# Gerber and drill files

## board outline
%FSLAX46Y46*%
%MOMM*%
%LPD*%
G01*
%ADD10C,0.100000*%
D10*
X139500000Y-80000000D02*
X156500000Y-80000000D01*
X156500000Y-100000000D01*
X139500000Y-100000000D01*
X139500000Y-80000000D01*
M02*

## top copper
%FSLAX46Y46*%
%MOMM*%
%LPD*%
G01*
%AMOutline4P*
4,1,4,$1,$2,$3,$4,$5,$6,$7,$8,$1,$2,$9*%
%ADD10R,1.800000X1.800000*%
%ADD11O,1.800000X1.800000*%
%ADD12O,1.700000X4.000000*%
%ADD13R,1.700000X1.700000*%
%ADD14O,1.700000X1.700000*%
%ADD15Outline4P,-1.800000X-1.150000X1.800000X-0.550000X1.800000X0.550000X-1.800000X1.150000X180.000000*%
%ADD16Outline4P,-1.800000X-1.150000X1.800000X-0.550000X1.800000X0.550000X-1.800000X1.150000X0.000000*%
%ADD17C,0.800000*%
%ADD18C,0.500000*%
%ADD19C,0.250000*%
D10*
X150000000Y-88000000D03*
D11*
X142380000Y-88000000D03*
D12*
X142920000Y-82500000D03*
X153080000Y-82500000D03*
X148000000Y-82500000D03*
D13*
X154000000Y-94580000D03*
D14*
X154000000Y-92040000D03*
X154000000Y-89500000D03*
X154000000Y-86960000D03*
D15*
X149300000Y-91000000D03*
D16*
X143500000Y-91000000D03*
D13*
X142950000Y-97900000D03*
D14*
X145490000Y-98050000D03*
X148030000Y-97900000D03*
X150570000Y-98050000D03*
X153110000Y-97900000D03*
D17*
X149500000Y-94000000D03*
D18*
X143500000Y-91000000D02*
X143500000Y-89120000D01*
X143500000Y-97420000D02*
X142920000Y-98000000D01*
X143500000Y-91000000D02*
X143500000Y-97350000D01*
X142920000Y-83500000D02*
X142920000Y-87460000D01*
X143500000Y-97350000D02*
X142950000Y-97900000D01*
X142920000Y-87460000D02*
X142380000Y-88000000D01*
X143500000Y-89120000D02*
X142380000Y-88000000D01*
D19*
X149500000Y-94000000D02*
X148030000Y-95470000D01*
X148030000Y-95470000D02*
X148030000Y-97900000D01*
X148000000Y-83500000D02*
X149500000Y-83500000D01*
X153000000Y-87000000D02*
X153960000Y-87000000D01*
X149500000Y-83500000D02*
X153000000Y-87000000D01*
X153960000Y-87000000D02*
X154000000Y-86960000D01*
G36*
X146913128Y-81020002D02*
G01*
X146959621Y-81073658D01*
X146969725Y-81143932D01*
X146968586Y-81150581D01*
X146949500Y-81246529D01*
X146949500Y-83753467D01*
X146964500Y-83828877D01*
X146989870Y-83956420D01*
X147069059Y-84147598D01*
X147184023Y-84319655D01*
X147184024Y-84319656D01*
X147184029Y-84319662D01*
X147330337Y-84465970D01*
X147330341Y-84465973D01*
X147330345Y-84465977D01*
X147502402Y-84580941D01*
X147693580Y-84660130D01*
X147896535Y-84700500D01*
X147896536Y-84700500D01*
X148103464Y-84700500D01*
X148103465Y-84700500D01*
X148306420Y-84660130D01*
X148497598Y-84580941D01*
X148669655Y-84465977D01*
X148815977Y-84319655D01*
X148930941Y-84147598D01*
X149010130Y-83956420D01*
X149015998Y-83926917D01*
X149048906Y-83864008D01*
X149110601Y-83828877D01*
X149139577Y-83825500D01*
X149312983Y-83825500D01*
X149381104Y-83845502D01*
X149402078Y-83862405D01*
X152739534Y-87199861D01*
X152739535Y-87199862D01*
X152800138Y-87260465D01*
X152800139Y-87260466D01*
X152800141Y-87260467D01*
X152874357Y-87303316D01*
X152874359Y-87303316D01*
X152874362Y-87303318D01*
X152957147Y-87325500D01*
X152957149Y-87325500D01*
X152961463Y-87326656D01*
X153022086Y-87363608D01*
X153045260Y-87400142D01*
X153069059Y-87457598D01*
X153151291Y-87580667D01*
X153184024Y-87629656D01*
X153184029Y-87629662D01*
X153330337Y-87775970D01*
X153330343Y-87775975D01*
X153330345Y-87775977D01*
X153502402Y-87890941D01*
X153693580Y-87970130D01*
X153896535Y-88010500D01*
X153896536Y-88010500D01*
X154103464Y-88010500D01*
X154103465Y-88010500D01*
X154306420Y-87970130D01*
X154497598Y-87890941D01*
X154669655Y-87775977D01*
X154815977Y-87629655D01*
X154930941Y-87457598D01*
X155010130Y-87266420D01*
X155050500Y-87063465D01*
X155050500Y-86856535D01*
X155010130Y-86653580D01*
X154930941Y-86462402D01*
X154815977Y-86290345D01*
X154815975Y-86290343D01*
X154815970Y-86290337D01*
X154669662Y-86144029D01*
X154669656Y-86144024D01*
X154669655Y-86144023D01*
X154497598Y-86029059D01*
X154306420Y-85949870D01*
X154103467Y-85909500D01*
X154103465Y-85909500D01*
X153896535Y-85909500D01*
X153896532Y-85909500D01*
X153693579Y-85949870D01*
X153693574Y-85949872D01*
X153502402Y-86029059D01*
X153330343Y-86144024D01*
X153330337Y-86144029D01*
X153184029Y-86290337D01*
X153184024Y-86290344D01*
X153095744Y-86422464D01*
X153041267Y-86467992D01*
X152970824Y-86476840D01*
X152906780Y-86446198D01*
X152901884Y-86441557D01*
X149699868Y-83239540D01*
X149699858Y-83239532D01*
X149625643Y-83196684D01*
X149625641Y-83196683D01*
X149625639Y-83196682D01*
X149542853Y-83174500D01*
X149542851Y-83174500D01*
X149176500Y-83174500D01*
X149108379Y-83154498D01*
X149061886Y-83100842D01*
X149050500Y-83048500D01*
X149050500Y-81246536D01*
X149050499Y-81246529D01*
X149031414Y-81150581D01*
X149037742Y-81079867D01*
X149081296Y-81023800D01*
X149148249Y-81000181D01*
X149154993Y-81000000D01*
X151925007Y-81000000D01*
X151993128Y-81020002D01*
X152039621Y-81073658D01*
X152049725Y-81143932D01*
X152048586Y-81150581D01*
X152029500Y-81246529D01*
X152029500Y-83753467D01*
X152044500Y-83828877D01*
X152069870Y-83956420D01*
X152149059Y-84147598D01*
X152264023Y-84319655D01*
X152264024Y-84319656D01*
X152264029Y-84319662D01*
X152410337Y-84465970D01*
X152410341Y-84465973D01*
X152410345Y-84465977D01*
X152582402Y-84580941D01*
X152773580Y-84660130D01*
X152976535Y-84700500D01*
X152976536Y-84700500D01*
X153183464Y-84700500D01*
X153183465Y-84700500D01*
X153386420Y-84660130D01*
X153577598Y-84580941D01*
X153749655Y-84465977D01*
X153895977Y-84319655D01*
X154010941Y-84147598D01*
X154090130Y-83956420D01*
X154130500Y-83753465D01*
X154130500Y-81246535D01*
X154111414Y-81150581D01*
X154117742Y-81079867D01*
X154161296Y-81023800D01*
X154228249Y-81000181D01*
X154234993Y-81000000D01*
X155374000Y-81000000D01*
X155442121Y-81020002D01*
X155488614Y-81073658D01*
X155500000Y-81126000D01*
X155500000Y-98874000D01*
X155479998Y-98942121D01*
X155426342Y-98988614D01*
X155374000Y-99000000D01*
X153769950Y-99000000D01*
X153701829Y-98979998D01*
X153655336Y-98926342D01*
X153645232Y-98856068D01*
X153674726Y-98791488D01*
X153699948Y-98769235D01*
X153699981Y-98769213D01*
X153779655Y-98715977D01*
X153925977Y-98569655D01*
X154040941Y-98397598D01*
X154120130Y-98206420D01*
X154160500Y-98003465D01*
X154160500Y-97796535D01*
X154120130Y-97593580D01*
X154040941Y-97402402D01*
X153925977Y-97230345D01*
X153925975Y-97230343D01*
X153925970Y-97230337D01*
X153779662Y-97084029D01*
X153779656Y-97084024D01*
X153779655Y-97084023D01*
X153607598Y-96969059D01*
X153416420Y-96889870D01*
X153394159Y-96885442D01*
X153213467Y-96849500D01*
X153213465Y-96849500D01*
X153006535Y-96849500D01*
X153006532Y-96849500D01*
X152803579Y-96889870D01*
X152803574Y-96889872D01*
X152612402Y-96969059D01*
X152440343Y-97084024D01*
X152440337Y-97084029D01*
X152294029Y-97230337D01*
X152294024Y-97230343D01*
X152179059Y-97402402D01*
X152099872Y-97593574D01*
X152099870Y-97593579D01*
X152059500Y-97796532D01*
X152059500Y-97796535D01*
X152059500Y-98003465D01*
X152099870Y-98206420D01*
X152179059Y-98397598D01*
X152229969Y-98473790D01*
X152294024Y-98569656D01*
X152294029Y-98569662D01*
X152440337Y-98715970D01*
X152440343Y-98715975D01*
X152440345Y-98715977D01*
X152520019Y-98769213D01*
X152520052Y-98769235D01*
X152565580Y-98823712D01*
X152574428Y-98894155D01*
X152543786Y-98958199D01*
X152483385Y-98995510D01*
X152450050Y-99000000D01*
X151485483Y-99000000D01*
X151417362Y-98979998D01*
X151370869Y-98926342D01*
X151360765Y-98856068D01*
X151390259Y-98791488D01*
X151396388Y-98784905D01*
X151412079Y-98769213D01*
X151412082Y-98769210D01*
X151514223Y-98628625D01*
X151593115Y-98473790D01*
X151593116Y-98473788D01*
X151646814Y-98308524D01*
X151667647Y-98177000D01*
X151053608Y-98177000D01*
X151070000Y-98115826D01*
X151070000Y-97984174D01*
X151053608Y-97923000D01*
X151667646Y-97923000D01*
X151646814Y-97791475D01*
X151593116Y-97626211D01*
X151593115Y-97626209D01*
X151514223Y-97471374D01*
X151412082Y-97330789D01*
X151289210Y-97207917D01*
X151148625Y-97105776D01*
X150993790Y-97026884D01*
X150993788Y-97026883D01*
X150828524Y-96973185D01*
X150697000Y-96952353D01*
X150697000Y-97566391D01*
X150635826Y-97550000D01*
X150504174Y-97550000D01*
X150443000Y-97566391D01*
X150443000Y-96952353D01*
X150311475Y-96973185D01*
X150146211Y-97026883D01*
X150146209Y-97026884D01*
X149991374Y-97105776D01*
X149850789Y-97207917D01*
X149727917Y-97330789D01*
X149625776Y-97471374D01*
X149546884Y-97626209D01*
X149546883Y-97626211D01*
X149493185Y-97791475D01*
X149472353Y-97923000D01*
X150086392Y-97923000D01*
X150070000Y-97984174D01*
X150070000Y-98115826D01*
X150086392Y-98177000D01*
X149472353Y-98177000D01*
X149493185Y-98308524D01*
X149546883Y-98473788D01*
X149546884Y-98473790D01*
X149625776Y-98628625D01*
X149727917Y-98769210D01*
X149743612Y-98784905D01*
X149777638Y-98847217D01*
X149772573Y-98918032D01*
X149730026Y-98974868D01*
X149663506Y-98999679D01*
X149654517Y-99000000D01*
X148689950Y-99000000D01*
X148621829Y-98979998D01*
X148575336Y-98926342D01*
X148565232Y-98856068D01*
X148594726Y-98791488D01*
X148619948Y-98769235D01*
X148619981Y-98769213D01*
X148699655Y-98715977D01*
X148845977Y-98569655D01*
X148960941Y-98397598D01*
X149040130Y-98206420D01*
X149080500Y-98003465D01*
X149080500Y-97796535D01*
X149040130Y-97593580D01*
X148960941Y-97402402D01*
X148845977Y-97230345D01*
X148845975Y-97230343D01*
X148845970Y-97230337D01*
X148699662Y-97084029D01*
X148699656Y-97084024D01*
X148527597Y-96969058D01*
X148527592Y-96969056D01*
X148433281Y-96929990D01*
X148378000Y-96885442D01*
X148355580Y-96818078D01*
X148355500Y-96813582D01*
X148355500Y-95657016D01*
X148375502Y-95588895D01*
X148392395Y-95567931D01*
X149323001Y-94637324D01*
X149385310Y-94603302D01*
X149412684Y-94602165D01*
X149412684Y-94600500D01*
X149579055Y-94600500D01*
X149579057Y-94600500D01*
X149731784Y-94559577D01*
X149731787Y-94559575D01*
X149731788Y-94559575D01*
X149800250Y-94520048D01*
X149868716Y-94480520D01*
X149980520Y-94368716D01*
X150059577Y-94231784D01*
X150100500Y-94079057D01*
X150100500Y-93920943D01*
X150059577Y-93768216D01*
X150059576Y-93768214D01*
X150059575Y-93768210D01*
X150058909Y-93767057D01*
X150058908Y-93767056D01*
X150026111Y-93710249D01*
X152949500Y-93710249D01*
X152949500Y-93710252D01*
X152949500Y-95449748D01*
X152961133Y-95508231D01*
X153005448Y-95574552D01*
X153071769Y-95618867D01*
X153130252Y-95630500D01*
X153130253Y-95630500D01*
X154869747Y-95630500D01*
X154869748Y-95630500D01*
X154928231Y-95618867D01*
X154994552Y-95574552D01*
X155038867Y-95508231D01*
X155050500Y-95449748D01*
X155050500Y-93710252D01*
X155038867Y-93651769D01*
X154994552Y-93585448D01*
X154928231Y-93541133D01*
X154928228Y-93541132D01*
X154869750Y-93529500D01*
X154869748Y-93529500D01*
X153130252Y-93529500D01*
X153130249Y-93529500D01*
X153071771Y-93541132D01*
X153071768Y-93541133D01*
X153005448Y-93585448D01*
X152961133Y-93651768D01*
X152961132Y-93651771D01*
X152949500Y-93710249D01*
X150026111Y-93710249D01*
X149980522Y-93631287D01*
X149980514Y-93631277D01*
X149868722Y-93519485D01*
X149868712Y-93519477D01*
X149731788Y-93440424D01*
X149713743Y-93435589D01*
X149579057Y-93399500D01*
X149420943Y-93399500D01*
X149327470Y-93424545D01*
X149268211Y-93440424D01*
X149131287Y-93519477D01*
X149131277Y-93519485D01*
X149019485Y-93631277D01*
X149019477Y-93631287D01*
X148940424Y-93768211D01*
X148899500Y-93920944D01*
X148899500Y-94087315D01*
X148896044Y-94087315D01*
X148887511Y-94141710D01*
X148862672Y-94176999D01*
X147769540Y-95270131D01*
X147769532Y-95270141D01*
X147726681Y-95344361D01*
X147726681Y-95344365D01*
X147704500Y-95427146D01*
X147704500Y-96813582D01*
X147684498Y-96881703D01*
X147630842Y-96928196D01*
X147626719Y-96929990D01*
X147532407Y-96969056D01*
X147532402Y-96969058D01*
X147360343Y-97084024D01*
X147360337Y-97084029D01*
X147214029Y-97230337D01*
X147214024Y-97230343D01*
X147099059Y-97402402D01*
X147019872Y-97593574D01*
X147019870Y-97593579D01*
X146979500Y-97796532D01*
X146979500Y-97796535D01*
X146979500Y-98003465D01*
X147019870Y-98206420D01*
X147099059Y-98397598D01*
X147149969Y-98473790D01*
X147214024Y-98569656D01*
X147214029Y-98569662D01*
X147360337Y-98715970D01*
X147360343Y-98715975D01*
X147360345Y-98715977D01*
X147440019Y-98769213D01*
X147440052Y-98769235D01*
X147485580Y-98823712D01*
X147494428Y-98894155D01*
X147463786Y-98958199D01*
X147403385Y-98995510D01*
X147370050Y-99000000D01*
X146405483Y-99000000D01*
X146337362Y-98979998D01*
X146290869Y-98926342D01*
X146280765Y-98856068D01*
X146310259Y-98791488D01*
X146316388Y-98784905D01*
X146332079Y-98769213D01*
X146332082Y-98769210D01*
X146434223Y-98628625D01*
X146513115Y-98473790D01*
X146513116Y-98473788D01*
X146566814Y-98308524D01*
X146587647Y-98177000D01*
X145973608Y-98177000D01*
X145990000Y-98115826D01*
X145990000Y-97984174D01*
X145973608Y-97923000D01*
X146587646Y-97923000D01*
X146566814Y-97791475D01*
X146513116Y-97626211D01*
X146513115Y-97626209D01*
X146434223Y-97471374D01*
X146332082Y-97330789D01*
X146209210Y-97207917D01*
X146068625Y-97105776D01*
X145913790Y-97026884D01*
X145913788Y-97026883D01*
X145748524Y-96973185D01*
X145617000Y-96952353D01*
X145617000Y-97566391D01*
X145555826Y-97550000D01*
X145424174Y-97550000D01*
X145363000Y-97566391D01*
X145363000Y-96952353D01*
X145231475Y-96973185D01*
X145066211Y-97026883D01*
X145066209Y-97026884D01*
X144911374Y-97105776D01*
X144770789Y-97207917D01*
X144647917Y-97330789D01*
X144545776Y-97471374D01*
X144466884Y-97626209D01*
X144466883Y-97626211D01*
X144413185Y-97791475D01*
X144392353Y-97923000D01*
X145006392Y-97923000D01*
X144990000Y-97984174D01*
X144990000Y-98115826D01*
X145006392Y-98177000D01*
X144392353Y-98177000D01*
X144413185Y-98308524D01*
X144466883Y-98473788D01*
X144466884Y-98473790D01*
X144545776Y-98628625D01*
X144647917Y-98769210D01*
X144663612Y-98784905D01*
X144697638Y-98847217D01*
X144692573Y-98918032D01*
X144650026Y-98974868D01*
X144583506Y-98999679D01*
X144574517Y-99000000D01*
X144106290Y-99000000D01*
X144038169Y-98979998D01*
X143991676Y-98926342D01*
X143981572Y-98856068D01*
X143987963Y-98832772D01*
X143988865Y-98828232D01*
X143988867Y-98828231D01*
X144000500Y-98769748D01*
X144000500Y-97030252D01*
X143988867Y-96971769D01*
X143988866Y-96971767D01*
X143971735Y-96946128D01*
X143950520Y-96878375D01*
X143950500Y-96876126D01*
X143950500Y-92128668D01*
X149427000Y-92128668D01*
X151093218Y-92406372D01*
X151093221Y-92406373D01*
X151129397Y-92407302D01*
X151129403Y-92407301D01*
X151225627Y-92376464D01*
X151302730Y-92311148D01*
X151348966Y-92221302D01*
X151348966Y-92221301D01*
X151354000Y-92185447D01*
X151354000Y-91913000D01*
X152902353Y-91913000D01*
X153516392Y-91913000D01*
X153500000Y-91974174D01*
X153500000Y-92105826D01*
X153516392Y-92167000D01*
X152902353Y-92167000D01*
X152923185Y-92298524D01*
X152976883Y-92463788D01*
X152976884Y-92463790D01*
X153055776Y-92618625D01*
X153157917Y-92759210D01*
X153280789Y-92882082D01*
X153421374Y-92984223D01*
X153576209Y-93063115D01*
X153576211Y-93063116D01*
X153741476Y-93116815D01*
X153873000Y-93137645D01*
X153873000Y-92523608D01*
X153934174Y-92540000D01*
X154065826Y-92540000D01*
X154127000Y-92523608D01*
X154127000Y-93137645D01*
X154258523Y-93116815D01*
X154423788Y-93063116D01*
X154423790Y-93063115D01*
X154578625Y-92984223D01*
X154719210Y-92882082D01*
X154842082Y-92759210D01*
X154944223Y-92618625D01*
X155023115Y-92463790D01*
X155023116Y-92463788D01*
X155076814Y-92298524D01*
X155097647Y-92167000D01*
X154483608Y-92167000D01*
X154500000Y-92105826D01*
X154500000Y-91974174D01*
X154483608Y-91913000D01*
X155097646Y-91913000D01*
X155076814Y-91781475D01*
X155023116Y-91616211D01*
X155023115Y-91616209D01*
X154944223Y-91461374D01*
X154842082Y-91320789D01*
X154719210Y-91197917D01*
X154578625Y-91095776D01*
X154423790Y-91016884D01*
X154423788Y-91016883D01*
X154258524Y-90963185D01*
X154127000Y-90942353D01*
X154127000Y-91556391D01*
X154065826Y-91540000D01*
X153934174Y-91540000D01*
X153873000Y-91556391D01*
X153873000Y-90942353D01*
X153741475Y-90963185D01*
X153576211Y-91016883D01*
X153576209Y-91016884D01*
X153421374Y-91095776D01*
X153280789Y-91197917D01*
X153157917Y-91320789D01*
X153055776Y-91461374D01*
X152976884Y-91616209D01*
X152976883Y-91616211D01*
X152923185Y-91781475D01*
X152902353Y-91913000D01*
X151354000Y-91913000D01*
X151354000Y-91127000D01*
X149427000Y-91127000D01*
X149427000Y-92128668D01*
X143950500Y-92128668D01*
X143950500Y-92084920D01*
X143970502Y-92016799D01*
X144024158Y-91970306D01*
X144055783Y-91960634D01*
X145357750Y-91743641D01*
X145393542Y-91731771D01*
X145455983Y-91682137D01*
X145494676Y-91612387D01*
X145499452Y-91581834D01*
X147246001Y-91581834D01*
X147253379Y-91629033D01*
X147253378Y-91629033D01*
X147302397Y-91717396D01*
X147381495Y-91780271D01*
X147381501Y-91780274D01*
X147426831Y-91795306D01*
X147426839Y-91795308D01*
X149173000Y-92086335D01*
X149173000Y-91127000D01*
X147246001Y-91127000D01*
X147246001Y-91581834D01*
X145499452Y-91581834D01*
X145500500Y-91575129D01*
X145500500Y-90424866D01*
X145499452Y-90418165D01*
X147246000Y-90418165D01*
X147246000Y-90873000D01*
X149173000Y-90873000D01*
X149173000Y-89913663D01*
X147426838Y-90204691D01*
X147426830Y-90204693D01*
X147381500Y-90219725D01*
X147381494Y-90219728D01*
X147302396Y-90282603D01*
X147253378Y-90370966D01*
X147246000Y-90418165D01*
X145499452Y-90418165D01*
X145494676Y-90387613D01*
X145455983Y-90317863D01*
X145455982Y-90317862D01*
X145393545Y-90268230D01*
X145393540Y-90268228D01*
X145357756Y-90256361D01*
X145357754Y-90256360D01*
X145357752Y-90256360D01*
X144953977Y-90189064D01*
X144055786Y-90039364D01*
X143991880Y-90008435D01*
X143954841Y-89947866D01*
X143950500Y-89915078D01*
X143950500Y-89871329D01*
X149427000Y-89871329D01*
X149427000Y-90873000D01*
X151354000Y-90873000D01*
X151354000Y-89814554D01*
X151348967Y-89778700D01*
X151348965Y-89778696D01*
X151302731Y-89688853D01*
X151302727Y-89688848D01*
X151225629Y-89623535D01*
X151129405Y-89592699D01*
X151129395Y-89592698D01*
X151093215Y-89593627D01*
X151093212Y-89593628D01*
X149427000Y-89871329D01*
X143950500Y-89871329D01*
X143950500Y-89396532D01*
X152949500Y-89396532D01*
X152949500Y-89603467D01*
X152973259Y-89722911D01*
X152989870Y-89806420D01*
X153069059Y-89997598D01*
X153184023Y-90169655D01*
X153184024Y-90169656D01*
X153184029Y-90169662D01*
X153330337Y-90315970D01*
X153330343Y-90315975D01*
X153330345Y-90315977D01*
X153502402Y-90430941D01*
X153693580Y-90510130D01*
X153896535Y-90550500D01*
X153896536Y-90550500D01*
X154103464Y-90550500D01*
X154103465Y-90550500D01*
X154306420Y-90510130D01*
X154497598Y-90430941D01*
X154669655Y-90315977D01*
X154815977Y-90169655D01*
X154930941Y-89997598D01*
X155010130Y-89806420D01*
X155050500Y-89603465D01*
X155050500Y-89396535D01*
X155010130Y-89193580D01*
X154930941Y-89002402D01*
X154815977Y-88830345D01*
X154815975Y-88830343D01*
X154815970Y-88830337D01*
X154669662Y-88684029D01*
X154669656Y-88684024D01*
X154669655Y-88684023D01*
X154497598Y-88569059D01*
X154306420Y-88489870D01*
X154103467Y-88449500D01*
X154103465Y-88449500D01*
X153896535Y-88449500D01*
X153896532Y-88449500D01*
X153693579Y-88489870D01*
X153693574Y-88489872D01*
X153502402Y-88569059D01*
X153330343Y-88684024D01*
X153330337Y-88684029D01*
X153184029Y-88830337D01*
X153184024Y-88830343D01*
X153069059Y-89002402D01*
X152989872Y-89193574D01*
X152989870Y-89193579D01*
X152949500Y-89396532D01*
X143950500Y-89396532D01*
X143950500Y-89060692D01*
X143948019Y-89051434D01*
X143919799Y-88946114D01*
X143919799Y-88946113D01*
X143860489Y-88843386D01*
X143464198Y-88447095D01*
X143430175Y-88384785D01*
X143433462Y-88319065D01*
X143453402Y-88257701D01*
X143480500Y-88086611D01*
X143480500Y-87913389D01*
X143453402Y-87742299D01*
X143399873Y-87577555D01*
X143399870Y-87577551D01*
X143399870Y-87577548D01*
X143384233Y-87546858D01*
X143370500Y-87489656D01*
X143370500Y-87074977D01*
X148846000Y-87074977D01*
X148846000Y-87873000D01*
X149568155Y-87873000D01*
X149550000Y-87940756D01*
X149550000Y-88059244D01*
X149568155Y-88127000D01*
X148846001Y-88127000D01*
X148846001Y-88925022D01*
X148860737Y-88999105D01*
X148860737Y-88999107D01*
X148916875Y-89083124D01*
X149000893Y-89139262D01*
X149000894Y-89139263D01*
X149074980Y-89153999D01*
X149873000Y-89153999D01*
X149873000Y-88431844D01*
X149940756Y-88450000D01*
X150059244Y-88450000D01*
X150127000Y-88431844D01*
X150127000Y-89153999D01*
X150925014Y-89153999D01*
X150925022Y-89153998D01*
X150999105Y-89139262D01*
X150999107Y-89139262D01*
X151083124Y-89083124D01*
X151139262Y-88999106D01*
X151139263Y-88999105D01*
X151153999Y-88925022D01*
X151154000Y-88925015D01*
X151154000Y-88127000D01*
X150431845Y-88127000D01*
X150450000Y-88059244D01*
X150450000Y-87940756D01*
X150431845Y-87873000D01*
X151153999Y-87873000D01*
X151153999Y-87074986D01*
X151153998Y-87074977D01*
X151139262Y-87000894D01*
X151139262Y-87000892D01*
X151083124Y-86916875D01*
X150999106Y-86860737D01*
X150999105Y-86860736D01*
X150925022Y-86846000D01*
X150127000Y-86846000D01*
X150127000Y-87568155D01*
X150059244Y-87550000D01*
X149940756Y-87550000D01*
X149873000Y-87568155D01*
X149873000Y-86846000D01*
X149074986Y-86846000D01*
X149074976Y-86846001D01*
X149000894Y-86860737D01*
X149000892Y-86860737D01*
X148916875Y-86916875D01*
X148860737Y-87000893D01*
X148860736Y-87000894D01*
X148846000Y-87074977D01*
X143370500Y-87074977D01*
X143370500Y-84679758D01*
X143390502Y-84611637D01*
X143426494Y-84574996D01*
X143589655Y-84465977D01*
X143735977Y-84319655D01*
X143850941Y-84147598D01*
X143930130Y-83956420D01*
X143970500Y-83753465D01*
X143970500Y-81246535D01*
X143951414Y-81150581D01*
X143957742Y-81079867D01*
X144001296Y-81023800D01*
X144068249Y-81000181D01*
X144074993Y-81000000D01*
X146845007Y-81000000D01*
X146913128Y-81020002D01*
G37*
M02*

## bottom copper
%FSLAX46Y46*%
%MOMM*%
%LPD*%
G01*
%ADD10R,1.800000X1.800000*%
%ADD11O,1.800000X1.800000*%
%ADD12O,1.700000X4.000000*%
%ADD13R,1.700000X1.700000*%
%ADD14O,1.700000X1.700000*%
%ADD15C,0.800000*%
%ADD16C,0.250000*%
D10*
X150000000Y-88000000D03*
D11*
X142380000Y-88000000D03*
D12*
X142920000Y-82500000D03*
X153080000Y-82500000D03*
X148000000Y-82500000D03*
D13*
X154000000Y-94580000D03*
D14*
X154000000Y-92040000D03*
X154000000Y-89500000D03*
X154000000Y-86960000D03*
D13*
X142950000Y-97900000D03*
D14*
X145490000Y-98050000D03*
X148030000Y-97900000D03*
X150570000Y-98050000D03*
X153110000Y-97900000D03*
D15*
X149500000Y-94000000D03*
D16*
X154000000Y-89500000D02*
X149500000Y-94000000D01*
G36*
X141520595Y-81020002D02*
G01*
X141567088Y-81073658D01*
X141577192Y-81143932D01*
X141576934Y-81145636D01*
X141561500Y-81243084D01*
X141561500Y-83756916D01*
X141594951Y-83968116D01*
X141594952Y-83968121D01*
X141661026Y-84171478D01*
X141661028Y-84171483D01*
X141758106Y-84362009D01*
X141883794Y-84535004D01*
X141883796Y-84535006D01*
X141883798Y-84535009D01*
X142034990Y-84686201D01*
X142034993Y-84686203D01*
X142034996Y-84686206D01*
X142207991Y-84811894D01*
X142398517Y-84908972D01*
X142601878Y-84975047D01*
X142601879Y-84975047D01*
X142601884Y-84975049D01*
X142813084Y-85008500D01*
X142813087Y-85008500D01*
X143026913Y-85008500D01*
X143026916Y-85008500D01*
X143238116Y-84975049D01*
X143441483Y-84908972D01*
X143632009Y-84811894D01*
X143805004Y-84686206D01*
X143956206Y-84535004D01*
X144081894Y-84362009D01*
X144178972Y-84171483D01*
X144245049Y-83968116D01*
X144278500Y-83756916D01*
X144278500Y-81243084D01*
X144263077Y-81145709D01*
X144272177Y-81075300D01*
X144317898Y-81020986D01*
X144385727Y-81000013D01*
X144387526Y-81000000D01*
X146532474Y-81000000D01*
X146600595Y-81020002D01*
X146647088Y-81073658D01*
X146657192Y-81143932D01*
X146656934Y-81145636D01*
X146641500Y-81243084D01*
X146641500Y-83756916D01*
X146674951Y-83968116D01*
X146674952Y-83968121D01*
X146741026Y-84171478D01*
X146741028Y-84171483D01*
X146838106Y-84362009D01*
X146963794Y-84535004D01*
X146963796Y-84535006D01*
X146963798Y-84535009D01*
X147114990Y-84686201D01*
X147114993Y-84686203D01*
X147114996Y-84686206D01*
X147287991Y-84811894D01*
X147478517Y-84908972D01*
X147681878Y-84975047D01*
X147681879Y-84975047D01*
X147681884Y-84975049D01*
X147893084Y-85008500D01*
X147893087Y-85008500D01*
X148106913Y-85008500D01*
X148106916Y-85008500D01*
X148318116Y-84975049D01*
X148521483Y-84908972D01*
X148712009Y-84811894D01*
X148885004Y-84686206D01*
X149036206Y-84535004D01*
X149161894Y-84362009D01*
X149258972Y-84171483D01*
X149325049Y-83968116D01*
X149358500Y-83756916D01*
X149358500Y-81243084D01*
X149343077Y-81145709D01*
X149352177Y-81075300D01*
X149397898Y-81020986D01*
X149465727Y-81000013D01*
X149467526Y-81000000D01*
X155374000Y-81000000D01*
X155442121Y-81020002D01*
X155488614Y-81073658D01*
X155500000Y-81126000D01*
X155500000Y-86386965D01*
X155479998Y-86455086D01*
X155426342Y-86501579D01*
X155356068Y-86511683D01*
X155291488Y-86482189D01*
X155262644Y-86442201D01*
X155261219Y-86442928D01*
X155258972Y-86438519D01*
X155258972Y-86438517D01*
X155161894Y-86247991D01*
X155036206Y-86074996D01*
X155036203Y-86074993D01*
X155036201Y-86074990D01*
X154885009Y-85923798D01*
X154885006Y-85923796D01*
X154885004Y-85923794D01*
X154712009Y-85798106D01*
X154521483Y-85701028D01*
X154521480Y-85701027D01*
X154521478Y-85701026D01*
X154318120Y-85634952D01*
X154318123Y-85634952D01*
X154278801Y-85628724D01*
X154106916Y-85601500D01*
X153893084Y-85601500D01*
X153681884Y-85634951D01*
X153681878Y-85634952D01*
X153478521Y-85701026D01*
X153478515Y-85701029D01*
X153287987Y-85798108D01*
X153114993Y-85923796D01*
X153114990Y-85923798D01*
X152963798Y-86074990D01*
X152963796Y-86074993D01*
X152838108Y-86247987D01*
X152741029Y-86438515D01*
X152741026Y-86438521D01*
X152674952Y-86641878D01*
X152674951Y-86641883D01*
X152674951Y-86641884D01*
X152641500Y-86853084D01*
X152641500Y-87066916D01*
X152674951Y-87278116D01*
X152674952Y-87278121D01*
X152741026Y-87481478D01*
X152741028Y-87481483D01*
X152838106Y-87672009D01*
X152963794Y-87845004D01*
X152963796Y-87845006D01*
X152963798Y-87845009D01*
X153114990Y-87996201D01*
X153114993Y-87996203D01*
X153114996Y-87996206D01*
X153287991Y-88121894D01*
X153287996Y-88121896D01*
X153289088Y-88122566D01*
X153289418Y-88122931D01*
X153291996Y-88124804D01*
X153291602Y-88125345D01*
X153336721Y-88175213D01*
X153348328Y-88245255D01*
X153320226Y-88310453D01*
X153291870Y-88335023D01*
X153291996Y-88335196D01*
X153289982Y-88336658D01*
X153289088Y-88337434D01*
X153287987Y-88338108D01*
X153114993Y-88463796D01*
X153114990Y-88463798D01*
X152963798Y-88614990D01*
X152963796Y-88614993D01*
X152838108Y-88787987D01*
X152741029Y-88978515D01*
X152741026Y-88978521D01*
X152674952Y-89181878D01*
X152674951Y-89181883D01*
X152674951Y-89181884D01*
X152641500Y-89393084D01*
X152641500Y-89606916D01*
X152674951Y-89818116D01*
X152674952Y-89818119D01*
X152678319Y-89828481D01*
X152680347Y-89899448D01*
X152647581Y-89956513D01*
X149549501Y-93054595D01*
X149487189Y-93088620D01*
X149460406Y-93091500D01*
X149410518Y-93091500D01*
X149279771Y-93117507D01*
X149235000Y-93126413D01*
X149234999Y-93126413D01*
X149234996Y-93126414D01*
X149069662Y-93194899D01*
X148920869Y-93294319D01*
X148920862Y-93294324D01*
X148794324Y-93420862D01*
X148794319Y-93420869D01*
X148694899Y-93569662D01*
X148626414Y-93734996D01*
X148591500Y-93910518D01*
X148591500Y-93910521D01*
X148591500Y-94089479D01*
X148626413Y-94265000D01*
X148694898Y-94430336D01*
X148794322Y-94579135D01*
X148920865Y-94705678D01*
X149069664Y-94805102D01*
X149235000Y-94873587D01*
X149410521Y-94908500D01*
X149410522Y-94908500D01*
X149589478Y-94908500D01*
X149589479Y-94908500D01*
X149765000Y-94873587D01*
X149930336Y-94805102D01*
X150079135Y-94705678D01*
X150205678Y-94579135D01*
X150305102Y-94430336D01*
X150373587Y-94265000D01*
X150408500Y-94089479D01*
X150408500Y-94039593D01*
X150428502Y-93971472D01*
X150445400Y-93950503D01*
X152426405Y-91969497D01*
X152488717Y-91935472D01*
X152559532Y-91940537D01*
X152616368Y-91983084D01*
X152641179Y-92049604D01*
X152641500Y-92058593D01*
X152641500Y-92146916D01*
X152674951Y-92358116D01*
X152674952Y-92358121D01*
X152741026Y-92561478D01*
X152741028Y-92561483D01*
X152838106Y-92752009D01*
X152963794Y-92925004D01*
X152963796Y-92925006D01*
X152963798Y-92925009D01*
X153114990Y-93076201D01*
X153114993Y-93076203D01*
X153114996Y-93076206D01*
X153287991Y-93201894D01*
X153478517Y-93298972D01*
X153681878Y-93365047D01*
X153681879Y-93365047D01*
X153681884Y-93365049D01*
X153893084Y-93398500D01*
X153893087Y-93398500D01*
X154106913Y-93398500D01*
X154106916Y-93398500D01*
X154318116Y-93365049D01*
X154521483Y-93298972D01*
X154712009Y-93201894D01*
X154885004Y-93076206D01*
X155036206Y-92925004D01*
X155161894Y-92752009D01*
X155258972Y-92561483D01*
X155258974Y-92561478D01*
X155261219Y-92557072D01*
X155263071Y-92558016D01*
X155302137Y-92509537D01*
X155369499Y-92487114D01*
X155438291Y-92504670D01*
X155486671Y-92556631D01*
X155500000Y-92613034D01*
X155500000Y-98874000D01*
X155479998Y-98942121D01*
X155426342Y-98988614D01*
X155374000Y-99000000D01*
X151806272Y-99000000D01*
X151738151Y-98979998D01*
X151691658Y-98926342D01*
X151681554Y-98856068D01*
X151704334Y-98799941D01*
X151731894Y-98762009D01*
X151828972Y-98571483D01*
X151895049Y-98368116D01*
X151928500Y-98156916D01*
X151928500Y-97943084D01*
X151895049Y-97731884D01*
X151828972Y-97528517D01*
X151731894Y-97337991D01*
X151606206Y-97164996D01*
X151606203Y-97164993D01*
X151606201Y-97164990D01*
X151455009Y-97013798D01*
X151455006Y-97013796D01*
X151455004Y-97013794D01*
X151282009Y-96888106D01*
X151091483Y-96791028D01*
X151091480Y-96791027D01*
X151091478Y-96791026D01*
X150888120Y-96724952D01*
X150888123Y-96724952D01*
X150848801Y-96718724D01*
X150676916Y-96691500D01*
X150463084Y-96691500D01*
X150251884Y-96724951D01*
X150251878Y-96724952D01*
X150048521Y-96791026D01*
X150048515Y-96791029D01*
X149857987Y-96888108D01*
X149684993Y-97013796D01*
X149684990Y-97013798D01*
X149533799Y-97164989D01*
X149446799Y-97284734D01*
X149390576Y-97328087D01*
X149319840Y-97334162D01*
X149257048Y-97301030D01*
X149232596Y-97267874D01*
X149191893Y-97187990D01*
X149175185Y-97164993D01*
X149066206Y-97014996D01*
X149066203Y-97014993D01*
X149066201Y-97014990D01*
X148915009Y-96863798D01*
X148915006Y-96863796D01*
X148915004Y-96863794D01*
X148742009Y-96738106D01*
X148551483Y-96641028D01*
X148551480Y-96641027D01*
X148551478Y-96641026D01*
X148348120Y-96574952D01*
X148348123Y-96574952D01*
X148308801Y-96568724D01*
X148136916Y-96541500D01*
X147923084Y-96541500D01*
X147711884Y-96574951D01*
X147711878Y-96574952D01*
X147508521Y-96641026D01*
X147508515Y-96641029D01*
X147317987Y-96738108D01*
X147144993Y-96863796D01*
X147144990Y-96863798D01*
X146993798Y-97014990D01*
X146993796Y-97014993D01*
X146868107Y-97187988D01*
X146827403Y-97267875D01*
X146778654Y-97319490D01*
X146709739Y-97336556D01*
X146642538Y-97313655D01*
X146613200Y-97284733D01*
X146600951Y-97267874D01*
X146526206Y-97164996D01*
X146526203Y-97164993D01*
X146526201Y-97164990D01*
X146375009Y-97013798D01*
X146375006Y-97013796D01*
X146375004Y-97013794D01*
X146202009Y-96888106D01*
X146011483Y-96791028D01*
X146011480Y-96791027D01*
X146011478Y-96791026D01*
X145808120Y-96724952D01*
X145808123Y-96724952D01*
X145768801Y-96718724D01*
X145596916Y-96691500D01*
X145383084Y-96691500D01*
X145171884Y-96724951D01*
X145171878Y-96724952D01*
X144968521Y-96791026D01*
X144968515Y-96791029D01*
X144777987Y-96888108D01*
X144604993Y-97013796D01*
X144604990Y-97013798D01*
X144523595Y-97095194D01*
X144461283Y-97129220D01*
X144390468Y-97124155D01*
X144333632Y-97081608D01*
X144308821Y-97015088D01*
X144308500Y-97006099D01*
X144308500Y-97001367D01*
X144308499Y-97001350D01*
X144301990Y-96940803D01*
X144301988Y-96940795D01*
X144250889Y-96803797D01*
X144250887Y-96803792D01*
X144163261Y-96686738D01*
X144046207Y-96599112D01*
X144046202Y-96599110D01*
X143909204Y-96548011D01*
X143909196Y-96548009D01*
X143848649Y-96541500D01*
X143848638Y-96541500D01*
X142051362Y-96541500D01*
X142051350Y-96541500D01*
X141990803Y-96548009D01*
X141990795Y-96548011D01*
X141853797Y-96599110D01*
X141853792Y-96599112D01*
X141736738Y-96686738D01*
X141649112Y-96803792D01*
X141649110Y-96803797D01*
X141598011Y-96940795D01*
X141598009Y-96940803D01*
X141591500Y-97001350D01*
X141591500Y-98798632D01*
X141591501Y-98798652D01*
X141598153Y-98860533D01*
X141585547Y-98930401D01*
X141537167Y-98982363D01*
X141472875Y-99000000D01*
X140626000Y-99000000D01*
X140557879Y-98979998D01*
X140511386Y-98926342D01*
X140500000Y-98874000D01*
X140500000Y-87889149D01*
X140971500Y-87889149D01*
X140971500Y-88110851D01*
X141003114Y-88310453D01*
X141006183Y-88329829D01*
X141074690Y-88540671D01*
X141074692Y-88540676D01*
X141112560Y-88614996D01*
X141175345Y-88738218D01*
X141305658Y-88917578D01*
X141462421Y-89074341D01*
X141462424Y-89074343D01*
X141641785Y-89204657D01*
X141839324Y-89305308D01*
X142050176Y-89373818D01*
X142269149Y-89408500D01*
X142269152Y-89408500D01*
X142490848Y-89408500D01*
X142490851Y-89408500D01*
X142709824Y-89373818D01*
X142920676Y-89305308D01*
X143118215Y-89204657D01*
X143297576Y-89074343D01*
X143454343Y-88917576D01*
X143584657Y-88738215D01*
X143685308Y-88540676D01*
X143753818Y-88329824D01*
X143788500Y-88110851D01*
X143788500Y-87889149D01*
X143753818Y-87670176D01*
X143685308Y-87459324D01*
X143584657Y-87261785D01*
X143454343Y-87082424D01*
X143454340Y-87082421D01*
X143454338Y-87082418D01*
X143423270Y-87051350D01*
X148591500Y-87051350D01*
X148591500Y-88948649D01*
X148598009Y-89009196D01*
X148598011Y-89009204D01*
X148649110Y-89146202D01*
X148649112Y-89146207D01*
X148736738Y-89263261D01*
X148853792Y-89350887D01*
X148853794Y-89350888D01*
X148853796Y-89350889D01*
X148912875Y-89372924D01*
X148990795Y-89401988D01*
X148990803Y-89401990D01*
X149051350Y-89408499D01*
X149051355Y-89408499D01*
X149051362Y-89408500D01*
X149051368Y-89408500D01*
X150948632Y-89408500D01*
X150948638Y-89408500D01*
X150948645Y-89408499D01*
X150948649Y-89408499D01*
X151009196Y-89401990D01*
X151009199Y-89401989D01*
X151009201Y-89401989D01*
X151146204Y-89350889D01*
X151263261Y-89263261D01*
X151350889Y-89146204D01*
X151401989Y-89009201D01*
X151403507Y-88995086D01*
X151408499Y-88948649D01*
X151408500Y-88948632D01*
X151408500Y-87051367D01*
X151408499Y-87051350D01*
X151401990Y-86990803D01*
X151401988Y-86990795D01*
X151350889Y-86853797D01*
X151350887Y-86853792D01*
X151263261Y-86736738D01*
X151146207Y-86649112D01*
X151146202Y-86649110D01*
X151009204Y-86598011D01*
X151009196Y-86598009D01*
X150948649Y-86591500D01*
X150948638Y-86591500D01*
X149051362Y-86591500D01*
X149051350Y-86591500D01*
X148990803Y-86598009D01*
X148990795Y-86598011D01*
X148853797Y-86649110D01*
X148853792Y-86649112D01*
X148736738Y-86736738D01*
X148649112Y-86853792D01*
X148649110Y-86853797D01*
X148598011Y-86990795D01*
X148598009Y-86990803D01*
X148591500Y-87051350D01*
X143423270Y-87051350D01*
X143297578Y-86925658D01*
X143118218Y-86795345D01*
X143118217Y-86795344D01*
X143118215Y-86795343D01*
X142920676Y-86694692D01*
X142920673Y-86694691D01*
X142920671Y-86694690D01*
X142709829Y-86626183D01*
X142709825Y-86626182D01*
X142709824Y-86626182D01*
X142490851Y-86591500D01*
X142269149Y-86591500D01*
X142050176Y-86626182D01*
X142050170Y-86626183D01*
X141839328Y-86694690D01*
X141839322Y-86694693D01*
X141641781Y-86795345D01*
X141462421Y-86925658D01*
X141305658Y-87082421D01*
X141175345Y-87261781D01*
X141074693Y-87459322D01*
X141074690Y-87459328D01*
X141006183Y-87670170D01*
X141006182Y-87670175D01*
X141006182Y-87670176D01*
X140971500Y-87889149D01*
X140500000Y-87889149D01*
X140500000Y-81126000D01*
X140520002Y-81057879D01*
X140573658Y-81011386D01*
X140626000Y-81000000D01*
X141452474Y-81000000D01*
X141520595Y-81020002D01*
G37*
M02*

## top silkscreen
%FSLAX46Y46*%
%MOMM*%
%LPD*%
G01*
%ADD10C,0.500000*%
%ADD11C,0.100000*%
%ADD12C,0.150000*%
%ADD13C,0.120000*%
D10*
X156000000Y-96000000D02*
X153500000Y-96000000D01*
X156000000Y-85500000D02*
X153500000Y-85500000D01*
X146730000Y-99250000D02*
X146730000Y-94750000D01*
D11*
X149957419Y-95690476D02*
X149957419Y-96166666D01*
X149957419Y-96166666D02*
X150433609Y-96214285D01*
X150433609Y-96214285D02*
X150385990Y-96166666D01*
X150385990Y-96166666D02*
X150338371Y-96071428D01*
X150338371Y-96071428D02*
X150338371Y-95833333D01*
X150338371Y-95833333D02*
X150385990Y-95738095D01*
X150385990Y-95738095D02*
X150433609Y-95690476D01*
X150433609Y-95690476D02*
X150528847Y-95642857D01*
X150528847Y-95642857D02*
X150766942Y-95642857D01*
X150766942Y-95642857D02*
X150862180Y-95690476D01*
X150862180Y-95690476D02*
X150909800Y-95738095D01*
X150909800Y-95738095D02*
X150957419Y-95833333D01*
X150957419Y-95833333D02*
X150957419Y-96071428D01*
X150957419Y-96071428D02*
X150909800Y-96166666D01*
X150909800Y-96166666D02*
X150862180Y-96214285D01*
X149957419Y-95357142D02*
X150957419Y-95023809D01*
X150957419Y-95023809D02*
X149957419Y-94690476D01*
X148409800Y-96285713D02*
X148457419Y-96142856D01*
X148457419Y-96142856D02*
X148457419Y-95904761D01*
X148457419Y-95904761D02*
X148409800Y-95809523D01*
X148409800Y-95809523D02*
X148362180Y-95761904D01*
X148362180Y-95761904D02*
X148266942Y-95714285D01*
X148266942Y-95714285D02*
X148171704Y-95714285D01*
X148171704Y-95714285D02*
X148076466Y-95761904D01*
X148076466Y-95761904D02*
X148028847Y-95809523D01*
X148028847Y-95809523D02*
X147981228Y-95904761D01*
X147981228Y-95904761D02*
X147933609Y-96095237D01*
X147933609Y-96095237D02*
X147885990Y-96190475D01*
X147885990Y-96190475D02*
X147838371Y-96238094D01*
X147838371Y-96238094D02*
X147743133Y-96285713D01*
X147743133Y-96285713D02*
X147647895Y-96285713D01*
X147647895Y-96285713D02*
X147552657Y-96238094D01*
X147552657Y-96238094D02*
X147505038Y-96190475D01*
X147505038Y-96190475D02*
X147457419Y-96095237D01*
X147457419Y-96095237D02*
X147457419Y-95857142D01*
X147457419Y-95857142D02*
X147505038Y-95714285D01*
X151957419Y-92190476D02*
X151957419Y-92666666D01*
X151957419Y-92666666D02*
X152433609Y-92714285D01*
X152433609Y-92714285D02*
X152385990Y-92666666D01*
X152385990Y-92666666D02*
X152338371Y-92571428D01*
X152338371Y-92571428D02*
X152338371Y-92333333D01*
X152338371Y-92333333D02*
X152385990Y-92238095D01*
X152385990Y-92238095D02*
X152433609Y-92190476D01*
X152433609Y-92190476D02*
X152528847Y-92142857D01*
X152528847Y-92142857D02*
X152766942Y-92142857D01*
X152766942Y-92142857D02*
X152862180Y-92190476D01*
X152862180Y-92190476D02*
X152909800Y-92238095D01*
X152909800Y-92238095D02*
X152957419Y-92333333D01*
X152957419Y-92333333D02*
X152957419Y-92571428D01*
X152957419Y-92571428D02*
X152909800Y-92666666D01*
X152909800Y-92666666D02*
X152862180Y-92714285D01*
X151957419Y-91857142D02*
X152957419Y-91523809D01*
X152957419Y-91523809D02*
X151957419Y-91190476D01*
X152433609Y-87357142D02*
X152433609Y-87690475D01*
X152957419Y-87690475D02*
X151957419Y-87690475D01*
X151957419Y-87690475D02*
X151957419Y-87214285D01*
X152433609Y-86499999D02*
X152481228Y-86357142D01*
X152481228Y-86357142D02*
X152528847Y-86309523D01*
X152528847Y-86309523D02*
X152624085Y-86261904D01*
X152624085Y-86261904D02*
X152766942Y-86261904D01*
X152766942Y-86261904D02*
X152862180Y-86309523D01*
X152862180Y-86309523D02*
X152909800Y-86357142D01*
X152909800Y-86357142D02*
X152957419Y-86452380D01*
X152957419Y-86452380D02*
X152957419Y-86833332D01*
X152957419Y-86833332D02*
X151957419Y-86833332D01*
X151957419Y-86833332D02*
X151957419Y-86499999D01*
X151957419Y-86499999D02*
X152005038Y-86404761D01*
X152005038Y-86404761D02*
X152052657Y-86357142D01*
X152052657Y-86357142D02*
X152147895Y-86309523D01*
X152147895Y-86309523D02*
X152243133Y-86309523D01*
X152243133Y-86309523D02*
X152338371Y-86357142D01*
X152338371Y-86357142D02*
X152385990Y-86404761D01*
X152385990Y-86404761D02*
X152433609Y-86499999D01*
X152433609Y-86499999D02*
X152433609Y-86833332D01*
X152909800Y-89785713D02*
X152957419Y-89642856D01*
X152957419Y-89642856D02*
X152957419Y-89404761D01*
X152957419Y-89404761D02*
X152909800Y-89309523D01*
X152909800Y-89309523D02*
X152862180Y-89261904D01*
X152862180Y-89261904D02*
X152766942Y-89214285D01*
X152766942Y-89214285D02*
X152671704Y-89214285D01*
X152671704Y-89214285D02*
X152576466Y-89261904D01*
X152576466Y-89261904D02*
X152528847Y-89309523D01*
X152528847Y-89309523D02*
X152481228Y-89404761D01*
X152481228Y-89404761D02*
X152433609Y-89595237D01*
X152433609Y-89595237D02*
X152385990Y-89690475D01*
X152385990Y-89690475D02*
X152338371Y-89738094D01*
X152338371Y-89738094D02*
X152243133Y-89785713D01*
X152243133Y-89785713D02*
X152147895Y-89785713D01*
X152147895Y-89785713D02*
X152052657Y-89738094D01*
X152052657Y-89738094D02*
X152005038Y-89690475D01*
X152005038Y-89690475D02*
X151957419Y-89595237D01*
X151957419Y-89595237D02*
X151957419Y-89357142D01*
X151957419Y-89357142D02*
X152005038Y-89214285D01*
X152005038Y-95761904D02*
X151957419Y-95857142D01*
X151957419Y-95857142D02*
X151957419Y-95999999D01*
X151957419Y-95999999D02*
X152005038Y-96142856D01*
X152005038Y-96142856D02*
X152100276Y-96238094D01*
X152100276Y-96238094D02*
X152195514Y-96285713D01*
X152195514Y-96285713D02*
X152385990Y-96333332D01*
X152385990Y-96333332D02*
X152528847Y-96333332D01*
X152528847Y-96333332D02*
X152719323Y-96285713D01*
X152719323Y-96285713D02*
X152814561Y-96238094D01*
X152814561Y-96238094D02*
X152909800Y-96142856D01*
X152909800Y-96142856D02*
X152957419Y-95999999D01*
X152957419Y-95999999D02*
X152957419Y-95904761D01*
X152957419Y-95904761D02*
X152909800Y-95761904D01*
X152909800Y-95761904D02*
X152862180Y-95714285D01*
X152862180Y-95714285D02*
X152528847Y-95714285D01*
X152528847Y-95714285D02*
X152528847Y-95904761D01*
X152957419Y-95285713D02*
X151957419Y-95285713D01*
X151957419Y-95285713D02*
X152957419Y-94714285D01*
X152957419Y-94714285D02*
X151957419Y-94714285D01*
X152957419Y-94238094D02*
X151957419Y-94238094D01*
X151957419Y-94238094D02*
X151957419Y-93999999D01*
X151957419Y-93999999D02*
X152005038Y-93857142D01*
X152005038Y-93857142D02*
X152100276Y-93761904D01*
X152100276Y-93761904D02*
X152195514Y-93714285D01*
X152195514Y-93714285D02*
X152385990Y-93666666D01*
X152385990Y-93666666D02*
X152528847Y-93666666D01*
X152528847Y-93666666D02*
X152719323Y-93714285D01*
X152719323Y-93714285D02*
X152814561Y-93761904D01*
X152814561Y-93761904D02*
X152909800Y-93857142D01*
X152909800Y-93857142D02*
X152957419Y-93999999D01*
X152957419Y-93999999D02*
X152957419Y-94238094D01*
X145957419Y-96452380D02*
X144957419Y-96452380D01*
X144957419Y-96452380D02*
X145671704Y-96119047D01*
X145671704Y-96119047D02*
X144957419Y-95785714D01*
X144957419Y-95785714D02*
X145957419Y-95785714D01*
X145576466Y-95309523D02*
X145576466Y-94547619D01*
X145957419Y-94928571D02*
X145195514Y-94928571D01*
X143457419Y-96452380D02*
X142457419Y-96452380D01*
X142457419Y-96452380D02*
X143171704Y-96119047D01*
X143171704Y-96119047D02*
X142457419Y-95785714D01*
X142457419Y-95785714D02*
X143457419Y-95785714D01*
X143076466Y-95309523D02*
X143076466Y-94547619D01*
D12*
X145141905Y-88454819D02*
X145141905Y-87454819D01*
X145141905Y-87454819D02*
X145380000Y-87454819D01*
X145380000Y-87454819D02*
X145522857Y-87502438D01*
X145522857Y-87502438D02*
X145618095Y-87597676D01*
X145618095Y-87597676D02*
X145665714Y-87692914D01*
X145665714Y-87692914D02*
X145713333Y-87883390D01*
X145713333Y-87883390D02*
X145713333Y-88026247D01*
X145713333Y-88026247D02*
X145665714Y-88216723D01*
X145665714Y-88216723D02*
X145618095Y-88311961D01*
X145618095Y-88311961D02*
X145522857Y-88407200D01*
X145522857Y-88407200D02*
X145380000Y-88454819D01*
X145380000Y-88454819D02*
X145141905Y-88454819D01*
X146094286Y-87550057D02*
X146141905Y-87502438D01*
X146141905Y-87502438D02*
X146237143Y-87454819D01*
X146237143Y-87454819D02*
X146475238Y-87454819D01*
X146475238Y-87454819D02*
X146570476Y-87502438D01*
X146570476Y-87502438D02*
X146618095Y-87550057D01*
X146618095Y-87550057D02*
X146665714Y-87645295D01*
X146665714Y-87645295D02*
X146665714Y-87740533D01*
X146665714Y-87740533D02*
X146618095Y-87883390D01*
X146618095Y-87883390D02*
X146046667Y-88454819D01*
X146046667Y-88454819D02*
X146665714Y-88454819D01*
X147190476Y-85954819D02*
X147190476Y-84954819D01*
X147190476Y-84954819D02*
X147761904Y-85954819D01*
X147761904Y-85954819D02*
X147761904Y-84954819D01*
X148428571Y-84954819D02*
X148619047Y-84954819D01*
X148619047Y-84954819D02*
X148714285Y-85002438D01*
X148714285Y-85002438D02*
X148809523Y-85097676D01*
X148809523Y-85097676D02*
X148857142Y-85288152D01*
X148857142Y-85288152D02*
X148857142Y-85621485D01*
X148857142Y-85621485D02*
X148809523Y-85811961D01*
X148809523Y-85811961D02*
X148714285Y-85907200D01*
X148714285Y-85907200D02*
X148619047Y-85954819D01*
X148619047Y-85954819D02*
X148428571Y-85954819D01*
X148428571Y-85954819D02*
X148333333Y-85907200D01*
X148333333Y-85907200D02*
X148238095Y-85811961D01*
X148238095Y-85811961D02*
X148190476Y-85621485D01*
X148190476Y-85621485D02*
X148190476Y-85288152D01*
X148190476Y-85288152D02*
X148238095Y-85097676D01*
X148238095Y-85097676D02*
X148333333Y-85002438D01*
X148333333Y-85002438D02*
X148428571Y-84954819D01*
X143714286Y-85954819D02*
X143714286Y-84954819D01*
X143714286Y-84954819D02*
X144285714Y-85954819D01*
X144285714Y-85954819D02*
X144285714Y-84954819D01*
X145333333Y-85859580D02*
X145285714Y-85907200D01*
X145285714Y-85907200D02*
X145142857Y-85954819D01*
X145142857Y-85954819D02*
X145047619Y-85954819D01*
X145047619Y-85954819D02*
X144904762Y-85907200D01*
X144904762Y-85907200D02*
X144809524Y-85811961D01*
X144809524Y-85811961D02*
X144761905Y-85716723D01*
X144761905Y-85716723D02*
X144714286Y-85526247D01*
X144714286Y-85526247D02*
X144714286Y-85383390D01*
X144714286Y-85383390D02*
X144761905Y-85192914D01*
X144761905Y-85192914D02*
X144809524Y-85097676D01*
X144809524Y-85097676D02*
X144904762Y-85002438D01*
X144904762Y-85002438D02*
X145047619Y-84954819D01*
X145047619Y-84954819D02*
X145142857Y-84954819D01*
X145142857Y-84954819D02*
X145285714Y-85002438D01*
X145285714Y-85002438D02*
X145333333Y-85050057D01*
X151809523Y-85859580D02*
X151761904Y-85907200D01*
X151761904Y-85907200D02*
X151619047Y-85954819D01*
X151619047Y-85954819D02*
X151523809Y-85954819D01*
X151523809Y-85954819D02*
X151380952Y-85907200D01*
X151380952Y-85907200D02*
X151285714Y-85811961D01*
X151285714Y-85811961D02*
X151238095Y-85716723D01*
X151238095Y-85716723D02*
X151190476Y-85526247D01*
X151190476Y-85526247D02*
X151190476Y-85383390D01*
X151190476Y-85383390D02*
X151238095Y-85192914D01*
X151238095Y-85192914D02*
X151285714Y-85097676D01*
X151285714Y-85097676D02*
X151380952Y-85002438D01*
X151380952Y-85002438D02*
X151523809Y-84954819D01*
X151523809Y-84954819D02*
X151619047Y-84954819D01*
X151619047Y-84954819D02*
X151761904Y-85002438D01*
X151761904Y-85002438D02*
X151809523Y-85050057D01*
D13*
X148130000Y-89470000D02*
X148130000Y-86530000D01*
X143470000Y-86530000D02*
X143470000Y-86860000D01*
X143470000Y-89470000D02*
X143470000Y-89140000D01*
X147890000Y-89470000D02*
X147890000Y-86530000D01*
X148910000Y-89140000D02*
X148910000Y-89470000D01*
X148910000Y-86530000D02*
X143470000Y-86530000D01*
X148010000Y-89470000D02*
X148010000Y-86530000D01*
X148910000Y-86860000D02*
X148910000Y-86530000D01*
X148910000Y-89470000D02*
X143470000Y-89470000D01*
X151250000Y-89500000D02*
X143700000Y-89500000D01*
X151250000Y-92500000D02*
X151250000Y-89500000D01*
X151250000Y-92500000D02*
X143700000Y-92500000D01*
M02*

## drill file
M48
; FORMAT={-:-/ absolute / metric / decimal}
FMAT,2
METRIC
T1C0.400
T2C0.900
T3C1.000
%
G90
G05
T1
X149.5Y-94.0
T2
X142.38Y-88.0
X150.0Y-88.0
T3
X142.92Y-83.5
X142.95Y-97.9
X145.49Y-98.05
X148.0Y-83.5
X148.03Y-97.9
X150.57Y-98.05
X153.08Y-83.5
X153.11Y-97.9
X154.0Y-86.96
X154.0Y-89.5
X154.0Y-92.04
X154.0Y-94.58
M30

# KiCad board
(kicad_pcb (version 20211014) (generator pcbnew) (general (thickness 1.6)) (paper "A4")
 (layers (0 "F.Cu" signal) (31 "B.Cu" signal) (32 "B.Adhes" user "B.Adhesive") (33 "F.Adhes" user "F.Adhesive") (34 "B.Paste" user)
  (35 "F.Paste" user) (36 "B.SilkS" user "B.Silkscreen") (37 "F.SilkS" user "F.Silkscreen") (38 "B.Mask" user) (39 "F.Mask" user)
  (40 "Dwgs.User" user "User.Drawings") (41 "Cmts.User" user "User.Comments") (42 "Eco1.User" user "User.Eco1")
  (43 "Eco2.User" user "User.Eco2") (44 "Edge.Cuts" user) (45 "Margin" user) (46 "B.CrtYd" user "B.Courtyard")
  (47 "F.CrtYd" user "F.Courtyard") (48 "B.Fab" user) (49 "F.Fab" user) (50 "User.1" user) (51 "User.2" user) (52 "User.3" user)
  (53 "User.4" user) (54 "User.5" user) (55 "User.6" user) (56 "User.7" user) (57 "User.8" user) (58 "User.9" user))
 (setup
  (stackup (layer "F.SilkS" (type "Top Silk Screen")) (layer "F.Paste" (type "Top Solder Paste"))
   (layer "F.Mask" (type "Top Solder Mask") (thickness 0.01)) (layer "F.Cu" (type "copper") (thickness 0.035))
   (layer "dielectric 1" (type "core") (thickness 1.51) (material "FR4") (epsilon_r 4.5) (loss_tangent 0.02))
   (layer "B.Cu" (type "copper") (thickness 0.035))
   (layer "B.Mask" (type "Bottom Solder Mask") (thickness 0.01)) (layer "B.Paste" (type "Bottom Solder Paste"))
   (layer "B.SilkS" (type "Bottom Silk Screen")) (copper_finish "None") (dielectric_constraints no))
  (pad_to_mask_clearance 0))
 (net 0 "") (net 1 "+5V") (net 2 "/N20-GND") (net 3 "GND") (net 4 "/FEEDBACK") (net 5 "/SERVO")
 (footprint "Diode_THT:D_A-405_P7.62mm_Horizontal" (layer "F.Cu") (at 150 88 180)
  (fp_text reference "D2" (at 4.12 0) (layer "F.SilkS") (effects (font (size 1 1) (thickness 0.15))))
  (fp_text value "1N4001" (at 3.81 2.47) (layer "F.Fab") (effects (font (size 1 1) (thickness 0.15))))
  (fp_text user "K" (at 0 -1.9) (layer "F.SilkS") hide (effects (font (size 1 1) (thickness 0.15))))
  (fp_line (start 1.87 -1.47) (end 1.87 1.47) (layer "F.SilkS") (width 0.12))
  (fp_line (start 6.53 1.47) (end 6.53 1.14) (layer "F.SilkS") (width 0.12))
  (fp_line (start 6.53 -1.47) (end 6.53 -1.14) (layer "F.SilkS") (width 0.12))
  (fp_line (start 2.11 -1.47) (end 2.11 1.47) (layer "F.SilkS") (width 0.12))
  (fp_line (start 1.09 -1.14) (end 1.09 -1.47) (layer "F.SilkS") (width 0.12))
  (fp_line (start 1.09 1.47) (end 6.53 1.47) (layer "F.SilkS") (width 0.12))
  (fp_line (start 1.99 -1.47) (end 1.99 1.47) (layer "F.SilkS") (width 0.12))
  (fp_line (start 1.09 1.14) (end 1.09 1.47) (layer "F.SilkS") (width 0.12))
  (fp_line (start 1.09 -1.47) (end 6.53 -1.47) (layer "F.SilkS") (width 0.12))
  (pad "1" thru_hole rect (at 0 0 180) (size 1.8 1.8) (drill 0.9) (layers *.Cu *.Mask) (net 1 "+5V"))
  (pad "2" thru_hole oval (at 7.62 0 180) (size 1.8 1.8) (drill 0.9) (layers *.Cu *.Mask) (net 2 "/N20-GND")))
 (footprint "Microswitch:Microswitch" (layer "F.Cu") (at 153.08 83.5 -90)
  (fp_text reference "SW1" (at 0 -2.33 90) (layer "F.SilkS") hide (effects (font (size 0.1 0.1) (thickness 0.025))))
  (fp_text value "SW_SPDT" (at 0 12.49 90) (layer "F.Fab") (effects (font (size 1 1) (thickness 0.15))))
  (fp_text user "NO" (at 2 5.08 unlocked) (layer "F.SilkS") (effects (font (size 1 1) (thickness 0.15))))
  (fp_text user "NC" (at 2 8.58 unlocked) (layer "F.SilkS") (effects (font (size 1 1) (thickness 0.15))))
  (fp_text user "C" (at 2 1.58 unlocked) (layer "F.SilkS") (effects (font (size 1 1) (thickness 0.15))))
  (pad "1" thru_hole oval (at 0 10.16 270) (size 4 1.7) (drill 1 (offset -1 0)) (layers *.Cu *.Mask) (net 2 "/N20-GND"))
  (pad "2" thru_hole oval (at 0 0 270) (size 4 1.7) (drill 1 (offset -1 0)) (layers *.Cu *.Mask) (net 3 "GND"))
  (pad "3" thru_hole oval (at 0 5.08 270) (size 4 1.7) (drill 1 (offset -1 0)) (layers *.Cu *.Mask) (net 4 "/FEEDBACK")))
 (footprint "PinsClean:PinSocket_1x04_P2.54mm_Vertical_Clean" (layer "F.Cu") (at 154 94.58 180)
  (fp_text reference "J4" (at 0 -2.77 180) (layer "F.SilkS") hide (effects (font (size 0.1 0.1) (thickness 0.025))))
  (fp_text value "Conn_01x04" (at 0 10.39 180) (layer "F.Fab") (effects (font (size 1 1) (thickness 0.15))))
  (pad "1" thru_hole rect (at 0 0 180) (size 1.7 1.7) (drill 1) (layers *.Cu *.Mask) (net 3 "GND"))
  (pad "2" thru_hole oval (at 0 2.54 180) (size 1.7 1.7) (drill 1) (layers *.Cu *.Mask) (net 1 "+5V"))
  (pad "3" thru_hole oval (at 0 5.08 180) (size 1.7 1.7) (drill 1) (layers *.Cu *.Mask) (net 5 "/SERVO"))
  (pad "4" thru_hole oval (at 0 7.62 180) (size 1.7 1.7) (drill 1) (layers *.Cu *.Mask) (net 4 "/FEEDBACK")))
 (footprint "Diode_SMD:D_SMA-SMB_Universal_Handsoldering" (layer "F.Cu") (at 146.4 91 180)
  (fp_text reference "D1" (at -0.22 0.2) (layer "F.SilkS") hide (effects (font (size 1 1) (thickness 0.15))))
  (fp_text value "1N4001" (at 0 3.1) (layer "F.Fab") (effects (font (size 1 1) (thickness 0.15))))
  (fp_line (start -4.85 1.5) (end 2.7 1.5) (layer "F.SilkS") (width 0.12))
  (fp_line (start -4.85 -1.5) (end -4.85 1.5) (layer "F.SilkS") (width 0.12))
  (fp_line (start -4.85 -1.5) (end 2.7 -1.5) (layer "F.SilkS") (width 0.12))
  (pad "1" smd trapezoid (at -2.9 0 180) (size 3.6 1.7) (rect_delta 0.6 0) (layers "F.Cu" "F.Paste" "F.Mask") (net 1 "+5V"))
  (pad "2" smd trapezoid (at 2.9 0) (size 3.6 1.7) (rect_delta 0.6 0) (layers "F.Cu" "F.Paste" "F.Mask") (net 2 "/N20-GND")))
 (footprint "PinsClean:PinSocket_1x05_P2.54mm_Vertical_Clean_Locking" (layer "F.Cu") (at 142.95 97.975 90)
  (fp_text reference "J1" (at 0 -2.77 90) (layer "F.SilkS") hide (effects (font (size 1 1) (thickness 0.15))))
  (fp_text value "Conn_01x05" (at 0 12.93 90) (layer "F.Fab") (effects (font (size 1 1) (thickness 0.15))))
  (pad "1" thru_hole rect (at 0.075 0 90) (size 1.7 1.7) (drill 1) (layers *.Cu *.Mask) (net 2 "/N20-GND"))
  (pad "2" thru_hole oval (at -0.075 2.54 90) (size 1.7 1.7) (drill 1) (layers *.Cu *.Mask) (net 1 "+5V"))
  (pad "3" thru_hole oval (at 0.075 5.08 90) (size 1.7 1.7) (drill 1) (layers *.Cu *.Mask) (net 5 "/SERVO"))
  (pad "4" thru_hole oval (at -0.075 7.62 90) (size 1.7 1.7) (drill 1) (layers *.Cu *.Mask) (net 1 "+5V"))
  (pad "5" thru_hole oval (at 0.075 10.16 90) (size 1.7 1.7) (drill 1) (layers *.Cu *.Mask) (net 3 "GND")))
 (gr_line (start 156 96) (end 153.5 96) (layer "F.SilkS") (width 0.5))
 (gr_line (start 156 85.5) (end 153.5 85.5) (layer "F.SilkS") (width 0.5))
 (gr_line (start 146.73 99.25) (end 146.73 94.75) (layer "F.SilkS") (width 0.5))
 (gr_rect (start 139.5 80) (end 156.5 100) (layer "Edge.Cuts") (width 0.1) (fill none))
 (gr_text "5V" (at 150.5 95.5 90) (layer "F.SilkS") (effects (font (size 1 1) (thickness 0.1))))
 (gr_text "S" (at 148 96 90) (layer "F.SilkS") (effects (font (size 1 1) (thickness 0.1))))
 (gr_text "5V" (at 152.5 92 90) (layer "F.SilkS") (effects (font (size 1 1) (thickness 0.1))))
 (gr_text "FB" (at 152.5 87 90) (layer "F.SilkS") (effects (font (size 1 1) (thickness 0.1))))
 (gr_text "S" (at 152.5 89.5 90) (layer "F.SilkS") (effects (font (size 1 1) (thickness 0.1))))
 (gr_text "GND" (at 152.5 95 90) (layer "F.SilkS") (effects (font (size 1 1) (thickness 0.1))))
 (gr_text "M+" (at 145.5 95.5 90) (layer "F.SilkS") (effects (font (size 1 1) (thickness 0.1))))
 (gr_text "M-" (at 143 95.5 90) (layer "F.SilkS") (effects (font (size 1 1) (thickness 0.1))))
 (segment (start 143.5 91) (end 143.5 89.12) (width 0.5) (layer "F.Cu") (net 2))
 (segment (start 143.5 97.42) (end 142.92 98) (width 0.5) (layer "F.Cu") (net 2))
 (segment (start 143.5 91) (end 143.5 97.35) (width 0.5) (layer "F.Cu") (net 2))
 (segment (start 142.92 83.5) (end 142.92 87.46) (width 0.5) (layer "F.Cu") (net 2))
 (segment (start 143.5 97.35) (end 142.95 97.9) (width 0.5) (layer "F.Cu") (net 2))
 (segment (start 142.92 87.46) (end 142.38 88) (width 0.5) (layer "F.Cu") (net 2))
 (segment (start 143.5 89.12) (end 142.38 88) (width 0.5) (layer "F.Cu") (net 2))
 (segment (start 149.5 94) (end 148.03 95.47) (width 0.25) (layer "F.Cu") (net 5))
 (segment (start 148.03 95.47) (end 148.03 97.9) (width 0.25) (layer "F.Cu") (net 5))
 (via (at 149.5 94) (size 0.8) (drill 0.4) (layers "F.Cu" "B.Cu") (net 5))
 (segment (start 154 89.5) (end 149.5 94) (width 0.25) (layer "B.Cu") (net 5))
 (segment (start 148 83.5) (end 149.5 83.5) (width 0.25) (layer "F.Cu") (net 4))
 (segment (start 153 87) (end 153.96 87) (width 0.25) (layer "F.Cu") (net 4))
 (segment (start 149.5 83.5) (end 153 87) (width 0.25) (layer "F.Cu") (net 4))
 (segment (start 153.96 87) (end 154 86.96) (width 0.25) (layer "F.Cu") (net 4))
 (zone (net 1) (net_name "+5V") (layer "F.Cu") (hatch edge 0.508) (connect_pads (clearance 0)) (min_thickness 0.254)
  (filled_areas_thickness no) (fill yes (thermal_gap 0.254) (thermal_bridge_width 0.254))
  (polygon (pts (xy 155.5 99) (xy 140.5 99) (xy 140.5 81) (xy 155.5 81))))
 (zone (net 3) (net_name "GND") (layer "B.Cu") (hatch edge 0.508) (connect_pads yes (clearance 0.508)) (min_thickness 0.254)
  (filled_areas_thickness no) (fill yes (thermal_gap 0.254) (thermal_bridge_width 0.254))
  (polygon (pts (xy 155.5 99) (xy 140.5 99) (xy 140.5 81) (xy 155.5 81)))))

